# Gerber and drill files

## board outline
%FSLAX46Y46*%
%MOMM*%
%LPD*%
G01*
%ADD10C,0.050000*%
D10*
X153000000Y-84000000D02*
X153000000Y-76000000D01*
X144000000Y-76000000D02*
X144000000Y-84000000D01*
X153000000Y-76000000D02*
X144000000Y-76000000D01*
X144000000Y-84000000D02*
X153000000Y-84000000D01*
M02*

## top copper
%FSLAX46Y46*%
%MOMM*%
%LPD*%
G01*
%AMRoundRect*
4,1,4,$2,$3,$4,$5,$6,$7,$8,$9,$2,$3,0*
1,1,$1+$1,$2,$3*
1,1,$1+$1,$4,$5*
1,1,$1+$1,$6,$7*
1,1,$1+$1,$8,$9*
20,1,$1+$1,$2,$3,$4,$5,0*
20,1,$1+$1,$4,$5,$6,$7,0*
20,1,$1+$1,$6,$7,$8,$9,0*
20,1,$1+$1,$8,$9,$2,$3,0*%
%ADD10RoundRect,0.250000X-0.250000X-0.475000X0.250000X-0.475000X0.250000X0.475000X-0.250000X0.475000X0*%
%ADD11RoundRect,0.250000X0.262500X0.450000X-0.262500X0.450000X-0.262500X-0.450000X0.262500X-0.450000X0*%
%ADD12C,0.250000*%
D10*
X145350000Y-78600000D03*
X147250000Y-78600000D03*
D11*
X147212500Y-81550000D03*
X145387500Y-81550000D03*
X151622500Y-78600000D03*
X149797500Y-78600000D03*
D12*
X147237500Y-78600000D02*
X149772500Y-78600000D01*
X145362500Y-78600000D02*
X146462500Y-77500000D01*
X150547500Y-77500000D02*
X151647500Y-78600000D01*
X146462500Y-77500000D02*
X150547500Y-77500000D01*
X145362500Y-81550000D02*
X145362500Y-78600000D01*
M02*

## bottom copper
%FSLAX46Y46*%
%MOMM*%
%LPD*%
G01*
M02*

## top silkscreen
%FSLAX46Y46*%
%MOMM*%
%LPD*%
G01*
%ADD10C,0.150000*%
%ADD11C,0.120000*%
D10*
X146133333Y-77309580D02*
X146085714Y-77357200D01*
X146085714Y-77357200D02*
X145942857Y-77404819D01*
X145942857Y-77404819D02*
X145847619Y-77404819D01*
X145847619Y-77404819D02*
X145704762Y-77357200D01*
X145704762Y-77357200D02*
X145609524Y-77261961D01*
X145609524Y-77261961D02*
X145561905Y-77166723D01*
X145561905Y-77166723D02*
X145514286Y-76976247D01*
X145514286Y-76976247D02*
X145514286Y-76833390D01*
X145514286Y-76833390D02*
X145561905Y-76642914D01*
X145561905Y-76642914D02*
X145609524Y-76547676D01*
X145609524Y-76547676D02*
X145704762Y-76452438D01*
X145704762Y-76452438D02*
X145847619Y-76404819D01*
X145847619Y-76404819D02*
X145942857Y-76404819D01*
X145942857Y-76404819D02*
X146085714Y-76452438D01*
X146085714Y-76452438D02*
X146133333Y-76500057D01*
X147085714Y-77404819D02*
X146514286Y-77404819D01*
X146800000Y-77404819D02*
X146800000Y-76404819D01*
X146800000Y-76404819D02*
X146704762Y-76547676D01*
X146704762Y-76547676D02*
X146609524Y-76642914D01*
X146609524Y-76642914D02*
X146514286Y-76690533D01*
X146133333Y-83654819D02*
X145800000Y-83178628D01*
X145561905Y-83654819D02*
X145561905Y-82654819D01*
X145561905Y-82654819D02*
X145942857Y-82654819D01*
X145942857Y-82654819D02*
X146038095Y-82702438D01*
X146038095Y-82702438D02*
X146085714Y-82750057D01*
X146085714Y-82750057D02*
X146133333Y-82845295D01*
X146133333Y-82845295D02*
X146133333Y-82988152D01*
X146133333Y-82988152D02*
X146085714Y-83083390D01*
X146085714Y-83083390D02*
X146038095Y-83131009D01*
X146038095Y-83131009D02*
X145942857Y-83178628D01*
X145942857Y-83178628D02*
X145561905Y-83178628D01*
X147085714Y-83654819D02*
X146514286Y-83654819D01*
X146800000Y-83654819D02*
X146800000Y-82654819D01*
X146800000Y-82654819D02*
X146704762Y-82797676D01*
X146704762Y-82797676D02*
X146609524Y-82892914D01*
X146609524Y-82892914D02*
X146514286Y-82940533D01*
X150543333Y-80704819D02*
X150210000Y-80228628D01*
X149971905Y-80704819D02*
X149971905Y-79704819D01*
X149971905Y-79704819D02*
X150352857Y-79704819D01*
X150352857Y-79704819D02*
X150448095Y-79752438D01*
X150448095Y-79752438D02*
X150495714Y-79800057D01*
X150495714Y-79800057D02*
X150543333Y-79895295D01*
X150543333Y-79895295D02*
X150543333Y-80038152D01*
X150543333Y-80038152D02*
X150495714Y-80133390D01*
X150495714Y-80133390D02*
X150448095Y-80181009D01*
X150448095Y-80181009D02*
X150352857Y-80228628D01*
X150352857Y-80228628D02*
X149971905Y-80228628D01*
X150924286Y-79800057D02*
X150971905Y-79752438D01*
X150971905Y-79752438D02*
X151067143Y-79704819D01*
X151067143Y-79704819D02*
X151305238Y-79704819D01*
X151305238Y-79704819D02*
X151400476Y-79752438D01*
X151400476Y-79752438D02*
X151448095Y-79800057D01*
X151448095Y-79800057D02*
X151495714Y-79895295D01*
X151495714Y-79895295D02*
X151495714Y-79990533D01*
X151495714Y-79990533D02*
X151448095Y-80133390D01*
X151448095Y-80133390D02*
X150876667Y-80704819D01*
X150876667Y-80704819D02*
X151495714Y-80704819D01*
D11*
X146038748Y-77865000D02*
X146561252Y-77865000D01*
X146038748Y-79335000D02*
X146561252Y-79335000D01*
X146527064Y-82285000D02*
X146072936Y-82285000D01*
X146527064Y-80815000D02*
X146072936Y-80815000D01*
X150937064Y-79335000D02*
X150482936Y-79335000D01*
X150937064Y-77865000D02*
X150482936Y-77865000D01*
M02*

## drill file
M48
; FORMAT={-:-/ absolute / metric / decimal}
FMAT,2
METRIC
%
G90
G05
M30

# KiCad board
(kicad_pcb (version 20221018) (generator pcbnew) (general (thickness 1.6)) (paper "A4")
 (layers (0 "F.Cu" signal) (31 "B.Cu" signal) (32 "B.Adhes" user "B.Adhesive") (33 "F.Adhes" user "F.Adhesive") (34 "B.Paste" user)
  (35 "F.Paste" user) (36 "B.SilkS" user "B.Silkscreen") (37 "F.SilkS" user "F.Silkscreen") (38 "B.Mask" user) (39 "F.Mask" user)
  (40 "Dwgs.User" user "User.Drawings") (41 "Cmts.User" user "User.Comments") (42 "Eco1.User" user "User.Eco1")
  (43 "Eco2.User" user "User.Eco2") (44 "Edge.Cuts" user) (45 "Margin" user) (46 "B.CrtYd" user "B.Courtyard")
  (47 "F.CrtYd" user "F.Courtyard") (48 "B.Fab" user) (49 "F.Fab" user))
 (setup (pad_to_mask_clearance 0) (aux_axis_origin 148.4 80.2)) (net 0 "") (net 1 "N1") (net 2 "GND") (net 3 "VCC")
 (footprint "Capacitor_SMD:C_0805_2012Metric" (layer "F.Cu") (at 146.3 78.6)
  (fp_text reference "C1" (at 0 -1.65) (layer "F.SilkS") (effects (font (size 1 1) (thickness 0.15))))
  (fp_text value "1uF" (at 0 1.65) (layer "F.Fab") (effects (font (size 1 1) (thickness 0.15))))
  (fp_line (start -0.261252 -0.735) (end 0.261252 -0.735) (stroke (width 0.12) (type solid)) (layer "F.SilkS"))
  (fp_line (start -0.261252 0.735) (end 0.261252 0.735) (stroke (width 0.12) (type solid)) (layer "F.SilkS"))
  (pad "1" smd roundrect (at -0.95 0) (size 1 1.45) (layers "F.Cu" "F.Paste" "F.Mask") (roundrect_rratio 0.25) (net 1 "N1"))
  (pad "2" smd roundrect (at 0.95 0) (size 1 1.45) (layers "F.Cu" "F.Paste" "F.Mask") (roundrect_rratio 0.25) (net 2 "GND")))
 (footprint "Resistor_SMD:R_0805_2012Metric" (layer "F.Cu") (at 146.3 81.55 180)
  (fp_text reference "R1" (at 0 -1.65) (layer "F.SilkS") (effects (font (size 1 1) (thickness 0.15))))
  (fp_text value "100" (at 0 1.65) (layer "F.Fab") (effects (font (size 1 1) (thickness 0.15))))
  (fp_line (start -0.227064 -0.735) (end 0.227064 -0.735) (stroke (width 0.12) (type solid)) (layer "F.SilkS"))
  (fp_line (start -0.227064 0.735) (end 0.227064 0.735) (stroke (width 0.12) (type solid)) (layer "F.SilkS"))
  (pad "1" smd roundrect (at -0.9125 0 180) (size 1.025 1.4) (layers "F.Cu" "F.Paste" "F.Mask") (roundrect_rratio 0.243902) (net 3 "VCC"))
  (pad "2" smd roundrect (at 0.9125 0 180) (size 1.025 1.4) (layers "F.Cu" "F.Paste" "F.Mask") (roundrect_rratio 0.243902) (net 1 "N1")))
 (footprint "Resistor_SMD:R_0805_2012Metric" (layer "F.Cu") (at 150.71 78.6 180)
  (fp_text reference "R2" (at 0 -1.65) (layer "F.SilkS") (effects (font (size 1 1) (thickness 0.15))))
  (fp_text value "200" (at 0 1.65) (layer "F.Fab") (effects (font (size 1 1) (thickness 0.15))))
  (fp_line (start -0.227064 -0.735) (end 0.227064 -0.735) (stroke (width 0.12) (type solid)) (layer "F.SilkS"))
  (fp_line (start -0.227064 0.735) (end 0.227064 0.735) (stroke (width 0.12) (type solid)) (layer "F.SilkS"))
  (pad "1" smd roundrect (at -0.9125 0 180) (size 1.025 1.4) (layers "F.Cu" "F.Paste" "F.Mask") (roundrect_rratio 0.243902) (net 1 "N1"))
  (pad "2" smd roundrect (at 0.9125 0 180) (size 1.025 1.4) (layers "F.Cu" "F.Paste" "F.Mask") (roundrect_rratio 0.243902) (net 2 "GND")))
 (gr_line (start 153 84) (end 153 76) (stroke (width 0.05) (type solid)) (layer "Edge.Cuts"))
 (gr_line (start 144 76) (end 144 84) (stroke (width 0.05) (type solid)) (layer "Edge.Cuts"))
 (gr_line (start 153 76) (end 144 76) (stroke (width 0.05) (type solid)) (layer "Edge.Cuts"))
 (gr_line (start 144 84) (end 153 84) (stroke (width 0.05) (type solid)) (layer "Edge.Cuts"))
 (segment (start 147.2375 78.6) (end 149.7725 78.6) (width 0.25) (layer "F.Cu") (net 2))
 (segment (start 145.3625 78.6) (end 146.4625 77.5) (width 0.25) (layer "F.Cu") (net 1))
 (segment (start 150.5475 77.5) (end 151.6475 78.6) (width 0.25) (layer "F.Cu") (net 1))
 (segment (start 146.4625 77.5) (end 150.5475 77.5) (width 0.25) (layer "F.Cu") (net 1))
 (segment (start 145.3625 81.55) (end 145.3625 78.6) (width 0.25) (layer "F.Cu") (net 1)))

